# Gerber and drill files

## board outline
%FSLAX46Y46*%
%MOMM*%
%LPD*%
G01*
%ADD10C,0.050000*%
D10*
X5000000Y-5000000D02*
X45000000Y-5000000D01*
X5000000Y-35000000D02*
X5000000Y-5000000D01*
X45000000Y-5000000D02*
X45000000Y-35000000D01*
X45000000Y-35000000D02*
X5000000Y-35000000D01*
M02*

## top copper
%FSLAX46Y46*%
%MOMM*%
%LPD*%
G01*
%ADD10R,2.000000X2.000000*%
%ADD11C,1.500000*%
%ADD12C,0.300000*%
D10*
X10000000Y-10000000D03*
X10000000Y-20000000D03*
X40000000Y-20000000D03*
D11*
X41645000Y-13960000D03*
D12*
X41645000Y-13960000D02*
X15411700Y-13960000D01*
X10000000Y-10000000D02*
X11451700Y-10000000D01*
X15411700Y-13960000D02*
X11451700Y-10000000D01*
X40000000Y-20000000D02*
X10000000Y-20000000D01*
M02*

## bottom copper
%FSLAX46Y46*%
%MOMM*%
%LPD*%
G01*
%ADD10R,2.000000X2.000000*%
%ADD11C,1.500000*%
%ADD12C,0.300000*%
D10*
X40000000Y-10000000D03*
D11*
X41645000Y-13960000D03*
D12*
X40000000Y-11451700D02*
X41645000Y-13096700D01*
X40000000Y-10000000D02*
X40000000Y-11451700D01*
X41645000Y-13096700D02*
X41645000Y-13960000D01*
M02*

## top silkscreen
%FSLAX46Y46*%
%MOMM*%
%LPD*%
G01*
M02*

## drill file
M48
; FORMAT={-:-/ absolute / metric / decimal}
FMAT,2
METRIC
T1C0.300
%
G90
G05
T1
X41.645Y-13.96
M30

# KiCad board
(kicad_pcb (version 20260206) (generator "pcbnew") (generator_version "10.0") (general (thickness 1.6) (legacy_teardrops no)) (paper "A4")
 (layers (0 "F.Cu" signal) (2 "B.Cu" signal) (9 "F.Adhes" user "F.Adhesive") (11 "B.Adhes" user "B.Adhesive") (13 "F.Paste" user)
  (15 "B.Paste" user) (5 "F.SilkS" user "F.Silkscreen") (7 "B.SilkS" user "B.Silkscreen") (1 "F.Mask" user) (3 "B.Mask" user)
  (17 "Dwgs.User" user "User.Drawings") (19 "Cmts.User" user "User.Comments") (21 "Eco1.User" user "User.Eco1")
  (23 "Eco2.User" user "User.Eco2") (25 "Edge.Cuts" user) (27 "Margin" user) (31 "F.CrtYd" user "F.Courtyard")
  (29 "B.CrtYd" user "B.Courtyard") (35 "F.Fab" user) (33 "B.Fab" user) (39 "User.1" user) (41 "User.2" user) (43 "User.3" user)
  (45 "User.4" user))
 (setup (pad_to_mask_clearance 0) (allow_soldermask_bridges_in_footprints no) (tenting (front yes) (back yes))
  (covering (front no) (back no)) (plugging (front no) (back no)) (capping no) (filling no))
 (gr_line (start 5 5) (end 45 5) (stroke (width 0.05) (type default)) (layer "Edge.Cuts"))
 (gr_line (start 5 35) (end 5 5) (stroke (width 0.05) (type default)) (layer "Edge.Cuts"))
 (gr_line (start 45 5) (end 45 35) (stroke (width 0.05) (type default)) (layer "Edge.Cuts"))
 (gr_line (start 45 35) (end 5 35) (stroke (width 0.05) (type default)) (layer "Edge.Cuts"))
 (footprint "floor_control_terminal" (layer "F.Cu") (at 10 10)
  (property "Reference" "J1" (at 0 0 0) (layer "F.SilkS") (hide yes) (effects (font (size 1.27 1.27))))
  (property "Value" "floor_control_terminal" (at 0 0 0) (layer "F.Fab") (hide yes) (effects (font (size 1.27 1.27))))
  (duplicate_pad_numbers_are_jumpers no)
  (pad "1" smd rect (at 0 0) (size 2 2) (layers "F.Cu" "F.Paste" "F.Mask") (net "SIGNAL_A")))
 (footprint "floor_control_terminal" (layer "B.Cu") (at 40 10)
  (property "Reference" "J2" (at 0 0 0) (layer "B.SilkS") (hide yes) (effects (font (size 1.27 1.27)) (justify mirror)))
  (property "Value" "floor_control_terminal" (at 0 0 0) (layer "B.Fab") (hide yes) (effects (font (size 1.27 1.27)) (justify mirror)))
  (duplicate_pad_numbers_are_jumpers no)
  (pad "1" smd rect (at 0 0) (size 2 2) (layers "B.Cu" "B.Paste" "B.Mask") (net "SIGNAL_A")))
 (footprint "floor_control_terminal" (layer "F.Cu") (at 10 20)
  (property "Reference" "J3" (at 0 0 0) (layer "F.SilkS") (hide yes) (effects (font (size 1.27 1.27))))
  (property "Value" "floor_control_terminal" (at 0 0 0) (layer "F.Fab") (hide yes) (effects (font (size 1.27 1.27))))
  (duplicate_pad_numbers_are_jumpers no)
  (pad "1" smd rect (at 0 0) (size 2 2) (layers "F.Cu" "F.Paste" "F.Mask") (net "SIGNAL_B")))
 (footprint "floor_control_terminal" (layer "F.Cu") (at 40 20)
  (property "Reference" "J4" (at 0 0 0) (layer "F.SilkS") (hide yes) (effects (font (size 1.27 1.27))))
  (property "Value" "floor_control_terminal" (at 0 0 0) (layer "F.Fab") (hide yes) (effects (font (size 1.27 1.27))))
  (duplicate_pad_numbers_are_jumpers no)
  (pad "1" smd rect (at 0 0) (size 2 2) (layers "F.Cu" "F.Paste" "F.Mask") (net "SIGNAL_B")))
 (segment (start 41.645 13.96) (end 15.4117 13.96) (width 0.3) (layer "F.Cu") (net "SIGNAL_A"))
 (segment (start 10 10) (end 11.4517 10) (width 0.3) (layer "F.Cu") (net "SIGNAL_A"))
 (segment (start 15.4117 13.96) (end 11.4517 10) (width 0.3) (layer "F.Cu") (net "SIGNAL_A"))
 (via (at 41.645 13.96) (size 1.5) (drill 0.3) (layers "F.Cu" "B.Cu") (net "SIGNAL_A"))
 (segment (start 40 11.4517) (end 41.645 13.0967) (width 0.3) (layer "B.Cu") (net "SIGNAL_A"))
 (segment (start 40 10) (end 40 11.4517) (width 0.3) (layer "B.Cu") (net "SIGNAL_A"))
 (segment (start 41.645 13.0967) (end 41.645 13.96) (width 0.3) (layer "B.Cu") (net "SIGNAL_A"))
 (segment (start 40 20) (end 10 20) (width 0.3) (layer "F.Cu") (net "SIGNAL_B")))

